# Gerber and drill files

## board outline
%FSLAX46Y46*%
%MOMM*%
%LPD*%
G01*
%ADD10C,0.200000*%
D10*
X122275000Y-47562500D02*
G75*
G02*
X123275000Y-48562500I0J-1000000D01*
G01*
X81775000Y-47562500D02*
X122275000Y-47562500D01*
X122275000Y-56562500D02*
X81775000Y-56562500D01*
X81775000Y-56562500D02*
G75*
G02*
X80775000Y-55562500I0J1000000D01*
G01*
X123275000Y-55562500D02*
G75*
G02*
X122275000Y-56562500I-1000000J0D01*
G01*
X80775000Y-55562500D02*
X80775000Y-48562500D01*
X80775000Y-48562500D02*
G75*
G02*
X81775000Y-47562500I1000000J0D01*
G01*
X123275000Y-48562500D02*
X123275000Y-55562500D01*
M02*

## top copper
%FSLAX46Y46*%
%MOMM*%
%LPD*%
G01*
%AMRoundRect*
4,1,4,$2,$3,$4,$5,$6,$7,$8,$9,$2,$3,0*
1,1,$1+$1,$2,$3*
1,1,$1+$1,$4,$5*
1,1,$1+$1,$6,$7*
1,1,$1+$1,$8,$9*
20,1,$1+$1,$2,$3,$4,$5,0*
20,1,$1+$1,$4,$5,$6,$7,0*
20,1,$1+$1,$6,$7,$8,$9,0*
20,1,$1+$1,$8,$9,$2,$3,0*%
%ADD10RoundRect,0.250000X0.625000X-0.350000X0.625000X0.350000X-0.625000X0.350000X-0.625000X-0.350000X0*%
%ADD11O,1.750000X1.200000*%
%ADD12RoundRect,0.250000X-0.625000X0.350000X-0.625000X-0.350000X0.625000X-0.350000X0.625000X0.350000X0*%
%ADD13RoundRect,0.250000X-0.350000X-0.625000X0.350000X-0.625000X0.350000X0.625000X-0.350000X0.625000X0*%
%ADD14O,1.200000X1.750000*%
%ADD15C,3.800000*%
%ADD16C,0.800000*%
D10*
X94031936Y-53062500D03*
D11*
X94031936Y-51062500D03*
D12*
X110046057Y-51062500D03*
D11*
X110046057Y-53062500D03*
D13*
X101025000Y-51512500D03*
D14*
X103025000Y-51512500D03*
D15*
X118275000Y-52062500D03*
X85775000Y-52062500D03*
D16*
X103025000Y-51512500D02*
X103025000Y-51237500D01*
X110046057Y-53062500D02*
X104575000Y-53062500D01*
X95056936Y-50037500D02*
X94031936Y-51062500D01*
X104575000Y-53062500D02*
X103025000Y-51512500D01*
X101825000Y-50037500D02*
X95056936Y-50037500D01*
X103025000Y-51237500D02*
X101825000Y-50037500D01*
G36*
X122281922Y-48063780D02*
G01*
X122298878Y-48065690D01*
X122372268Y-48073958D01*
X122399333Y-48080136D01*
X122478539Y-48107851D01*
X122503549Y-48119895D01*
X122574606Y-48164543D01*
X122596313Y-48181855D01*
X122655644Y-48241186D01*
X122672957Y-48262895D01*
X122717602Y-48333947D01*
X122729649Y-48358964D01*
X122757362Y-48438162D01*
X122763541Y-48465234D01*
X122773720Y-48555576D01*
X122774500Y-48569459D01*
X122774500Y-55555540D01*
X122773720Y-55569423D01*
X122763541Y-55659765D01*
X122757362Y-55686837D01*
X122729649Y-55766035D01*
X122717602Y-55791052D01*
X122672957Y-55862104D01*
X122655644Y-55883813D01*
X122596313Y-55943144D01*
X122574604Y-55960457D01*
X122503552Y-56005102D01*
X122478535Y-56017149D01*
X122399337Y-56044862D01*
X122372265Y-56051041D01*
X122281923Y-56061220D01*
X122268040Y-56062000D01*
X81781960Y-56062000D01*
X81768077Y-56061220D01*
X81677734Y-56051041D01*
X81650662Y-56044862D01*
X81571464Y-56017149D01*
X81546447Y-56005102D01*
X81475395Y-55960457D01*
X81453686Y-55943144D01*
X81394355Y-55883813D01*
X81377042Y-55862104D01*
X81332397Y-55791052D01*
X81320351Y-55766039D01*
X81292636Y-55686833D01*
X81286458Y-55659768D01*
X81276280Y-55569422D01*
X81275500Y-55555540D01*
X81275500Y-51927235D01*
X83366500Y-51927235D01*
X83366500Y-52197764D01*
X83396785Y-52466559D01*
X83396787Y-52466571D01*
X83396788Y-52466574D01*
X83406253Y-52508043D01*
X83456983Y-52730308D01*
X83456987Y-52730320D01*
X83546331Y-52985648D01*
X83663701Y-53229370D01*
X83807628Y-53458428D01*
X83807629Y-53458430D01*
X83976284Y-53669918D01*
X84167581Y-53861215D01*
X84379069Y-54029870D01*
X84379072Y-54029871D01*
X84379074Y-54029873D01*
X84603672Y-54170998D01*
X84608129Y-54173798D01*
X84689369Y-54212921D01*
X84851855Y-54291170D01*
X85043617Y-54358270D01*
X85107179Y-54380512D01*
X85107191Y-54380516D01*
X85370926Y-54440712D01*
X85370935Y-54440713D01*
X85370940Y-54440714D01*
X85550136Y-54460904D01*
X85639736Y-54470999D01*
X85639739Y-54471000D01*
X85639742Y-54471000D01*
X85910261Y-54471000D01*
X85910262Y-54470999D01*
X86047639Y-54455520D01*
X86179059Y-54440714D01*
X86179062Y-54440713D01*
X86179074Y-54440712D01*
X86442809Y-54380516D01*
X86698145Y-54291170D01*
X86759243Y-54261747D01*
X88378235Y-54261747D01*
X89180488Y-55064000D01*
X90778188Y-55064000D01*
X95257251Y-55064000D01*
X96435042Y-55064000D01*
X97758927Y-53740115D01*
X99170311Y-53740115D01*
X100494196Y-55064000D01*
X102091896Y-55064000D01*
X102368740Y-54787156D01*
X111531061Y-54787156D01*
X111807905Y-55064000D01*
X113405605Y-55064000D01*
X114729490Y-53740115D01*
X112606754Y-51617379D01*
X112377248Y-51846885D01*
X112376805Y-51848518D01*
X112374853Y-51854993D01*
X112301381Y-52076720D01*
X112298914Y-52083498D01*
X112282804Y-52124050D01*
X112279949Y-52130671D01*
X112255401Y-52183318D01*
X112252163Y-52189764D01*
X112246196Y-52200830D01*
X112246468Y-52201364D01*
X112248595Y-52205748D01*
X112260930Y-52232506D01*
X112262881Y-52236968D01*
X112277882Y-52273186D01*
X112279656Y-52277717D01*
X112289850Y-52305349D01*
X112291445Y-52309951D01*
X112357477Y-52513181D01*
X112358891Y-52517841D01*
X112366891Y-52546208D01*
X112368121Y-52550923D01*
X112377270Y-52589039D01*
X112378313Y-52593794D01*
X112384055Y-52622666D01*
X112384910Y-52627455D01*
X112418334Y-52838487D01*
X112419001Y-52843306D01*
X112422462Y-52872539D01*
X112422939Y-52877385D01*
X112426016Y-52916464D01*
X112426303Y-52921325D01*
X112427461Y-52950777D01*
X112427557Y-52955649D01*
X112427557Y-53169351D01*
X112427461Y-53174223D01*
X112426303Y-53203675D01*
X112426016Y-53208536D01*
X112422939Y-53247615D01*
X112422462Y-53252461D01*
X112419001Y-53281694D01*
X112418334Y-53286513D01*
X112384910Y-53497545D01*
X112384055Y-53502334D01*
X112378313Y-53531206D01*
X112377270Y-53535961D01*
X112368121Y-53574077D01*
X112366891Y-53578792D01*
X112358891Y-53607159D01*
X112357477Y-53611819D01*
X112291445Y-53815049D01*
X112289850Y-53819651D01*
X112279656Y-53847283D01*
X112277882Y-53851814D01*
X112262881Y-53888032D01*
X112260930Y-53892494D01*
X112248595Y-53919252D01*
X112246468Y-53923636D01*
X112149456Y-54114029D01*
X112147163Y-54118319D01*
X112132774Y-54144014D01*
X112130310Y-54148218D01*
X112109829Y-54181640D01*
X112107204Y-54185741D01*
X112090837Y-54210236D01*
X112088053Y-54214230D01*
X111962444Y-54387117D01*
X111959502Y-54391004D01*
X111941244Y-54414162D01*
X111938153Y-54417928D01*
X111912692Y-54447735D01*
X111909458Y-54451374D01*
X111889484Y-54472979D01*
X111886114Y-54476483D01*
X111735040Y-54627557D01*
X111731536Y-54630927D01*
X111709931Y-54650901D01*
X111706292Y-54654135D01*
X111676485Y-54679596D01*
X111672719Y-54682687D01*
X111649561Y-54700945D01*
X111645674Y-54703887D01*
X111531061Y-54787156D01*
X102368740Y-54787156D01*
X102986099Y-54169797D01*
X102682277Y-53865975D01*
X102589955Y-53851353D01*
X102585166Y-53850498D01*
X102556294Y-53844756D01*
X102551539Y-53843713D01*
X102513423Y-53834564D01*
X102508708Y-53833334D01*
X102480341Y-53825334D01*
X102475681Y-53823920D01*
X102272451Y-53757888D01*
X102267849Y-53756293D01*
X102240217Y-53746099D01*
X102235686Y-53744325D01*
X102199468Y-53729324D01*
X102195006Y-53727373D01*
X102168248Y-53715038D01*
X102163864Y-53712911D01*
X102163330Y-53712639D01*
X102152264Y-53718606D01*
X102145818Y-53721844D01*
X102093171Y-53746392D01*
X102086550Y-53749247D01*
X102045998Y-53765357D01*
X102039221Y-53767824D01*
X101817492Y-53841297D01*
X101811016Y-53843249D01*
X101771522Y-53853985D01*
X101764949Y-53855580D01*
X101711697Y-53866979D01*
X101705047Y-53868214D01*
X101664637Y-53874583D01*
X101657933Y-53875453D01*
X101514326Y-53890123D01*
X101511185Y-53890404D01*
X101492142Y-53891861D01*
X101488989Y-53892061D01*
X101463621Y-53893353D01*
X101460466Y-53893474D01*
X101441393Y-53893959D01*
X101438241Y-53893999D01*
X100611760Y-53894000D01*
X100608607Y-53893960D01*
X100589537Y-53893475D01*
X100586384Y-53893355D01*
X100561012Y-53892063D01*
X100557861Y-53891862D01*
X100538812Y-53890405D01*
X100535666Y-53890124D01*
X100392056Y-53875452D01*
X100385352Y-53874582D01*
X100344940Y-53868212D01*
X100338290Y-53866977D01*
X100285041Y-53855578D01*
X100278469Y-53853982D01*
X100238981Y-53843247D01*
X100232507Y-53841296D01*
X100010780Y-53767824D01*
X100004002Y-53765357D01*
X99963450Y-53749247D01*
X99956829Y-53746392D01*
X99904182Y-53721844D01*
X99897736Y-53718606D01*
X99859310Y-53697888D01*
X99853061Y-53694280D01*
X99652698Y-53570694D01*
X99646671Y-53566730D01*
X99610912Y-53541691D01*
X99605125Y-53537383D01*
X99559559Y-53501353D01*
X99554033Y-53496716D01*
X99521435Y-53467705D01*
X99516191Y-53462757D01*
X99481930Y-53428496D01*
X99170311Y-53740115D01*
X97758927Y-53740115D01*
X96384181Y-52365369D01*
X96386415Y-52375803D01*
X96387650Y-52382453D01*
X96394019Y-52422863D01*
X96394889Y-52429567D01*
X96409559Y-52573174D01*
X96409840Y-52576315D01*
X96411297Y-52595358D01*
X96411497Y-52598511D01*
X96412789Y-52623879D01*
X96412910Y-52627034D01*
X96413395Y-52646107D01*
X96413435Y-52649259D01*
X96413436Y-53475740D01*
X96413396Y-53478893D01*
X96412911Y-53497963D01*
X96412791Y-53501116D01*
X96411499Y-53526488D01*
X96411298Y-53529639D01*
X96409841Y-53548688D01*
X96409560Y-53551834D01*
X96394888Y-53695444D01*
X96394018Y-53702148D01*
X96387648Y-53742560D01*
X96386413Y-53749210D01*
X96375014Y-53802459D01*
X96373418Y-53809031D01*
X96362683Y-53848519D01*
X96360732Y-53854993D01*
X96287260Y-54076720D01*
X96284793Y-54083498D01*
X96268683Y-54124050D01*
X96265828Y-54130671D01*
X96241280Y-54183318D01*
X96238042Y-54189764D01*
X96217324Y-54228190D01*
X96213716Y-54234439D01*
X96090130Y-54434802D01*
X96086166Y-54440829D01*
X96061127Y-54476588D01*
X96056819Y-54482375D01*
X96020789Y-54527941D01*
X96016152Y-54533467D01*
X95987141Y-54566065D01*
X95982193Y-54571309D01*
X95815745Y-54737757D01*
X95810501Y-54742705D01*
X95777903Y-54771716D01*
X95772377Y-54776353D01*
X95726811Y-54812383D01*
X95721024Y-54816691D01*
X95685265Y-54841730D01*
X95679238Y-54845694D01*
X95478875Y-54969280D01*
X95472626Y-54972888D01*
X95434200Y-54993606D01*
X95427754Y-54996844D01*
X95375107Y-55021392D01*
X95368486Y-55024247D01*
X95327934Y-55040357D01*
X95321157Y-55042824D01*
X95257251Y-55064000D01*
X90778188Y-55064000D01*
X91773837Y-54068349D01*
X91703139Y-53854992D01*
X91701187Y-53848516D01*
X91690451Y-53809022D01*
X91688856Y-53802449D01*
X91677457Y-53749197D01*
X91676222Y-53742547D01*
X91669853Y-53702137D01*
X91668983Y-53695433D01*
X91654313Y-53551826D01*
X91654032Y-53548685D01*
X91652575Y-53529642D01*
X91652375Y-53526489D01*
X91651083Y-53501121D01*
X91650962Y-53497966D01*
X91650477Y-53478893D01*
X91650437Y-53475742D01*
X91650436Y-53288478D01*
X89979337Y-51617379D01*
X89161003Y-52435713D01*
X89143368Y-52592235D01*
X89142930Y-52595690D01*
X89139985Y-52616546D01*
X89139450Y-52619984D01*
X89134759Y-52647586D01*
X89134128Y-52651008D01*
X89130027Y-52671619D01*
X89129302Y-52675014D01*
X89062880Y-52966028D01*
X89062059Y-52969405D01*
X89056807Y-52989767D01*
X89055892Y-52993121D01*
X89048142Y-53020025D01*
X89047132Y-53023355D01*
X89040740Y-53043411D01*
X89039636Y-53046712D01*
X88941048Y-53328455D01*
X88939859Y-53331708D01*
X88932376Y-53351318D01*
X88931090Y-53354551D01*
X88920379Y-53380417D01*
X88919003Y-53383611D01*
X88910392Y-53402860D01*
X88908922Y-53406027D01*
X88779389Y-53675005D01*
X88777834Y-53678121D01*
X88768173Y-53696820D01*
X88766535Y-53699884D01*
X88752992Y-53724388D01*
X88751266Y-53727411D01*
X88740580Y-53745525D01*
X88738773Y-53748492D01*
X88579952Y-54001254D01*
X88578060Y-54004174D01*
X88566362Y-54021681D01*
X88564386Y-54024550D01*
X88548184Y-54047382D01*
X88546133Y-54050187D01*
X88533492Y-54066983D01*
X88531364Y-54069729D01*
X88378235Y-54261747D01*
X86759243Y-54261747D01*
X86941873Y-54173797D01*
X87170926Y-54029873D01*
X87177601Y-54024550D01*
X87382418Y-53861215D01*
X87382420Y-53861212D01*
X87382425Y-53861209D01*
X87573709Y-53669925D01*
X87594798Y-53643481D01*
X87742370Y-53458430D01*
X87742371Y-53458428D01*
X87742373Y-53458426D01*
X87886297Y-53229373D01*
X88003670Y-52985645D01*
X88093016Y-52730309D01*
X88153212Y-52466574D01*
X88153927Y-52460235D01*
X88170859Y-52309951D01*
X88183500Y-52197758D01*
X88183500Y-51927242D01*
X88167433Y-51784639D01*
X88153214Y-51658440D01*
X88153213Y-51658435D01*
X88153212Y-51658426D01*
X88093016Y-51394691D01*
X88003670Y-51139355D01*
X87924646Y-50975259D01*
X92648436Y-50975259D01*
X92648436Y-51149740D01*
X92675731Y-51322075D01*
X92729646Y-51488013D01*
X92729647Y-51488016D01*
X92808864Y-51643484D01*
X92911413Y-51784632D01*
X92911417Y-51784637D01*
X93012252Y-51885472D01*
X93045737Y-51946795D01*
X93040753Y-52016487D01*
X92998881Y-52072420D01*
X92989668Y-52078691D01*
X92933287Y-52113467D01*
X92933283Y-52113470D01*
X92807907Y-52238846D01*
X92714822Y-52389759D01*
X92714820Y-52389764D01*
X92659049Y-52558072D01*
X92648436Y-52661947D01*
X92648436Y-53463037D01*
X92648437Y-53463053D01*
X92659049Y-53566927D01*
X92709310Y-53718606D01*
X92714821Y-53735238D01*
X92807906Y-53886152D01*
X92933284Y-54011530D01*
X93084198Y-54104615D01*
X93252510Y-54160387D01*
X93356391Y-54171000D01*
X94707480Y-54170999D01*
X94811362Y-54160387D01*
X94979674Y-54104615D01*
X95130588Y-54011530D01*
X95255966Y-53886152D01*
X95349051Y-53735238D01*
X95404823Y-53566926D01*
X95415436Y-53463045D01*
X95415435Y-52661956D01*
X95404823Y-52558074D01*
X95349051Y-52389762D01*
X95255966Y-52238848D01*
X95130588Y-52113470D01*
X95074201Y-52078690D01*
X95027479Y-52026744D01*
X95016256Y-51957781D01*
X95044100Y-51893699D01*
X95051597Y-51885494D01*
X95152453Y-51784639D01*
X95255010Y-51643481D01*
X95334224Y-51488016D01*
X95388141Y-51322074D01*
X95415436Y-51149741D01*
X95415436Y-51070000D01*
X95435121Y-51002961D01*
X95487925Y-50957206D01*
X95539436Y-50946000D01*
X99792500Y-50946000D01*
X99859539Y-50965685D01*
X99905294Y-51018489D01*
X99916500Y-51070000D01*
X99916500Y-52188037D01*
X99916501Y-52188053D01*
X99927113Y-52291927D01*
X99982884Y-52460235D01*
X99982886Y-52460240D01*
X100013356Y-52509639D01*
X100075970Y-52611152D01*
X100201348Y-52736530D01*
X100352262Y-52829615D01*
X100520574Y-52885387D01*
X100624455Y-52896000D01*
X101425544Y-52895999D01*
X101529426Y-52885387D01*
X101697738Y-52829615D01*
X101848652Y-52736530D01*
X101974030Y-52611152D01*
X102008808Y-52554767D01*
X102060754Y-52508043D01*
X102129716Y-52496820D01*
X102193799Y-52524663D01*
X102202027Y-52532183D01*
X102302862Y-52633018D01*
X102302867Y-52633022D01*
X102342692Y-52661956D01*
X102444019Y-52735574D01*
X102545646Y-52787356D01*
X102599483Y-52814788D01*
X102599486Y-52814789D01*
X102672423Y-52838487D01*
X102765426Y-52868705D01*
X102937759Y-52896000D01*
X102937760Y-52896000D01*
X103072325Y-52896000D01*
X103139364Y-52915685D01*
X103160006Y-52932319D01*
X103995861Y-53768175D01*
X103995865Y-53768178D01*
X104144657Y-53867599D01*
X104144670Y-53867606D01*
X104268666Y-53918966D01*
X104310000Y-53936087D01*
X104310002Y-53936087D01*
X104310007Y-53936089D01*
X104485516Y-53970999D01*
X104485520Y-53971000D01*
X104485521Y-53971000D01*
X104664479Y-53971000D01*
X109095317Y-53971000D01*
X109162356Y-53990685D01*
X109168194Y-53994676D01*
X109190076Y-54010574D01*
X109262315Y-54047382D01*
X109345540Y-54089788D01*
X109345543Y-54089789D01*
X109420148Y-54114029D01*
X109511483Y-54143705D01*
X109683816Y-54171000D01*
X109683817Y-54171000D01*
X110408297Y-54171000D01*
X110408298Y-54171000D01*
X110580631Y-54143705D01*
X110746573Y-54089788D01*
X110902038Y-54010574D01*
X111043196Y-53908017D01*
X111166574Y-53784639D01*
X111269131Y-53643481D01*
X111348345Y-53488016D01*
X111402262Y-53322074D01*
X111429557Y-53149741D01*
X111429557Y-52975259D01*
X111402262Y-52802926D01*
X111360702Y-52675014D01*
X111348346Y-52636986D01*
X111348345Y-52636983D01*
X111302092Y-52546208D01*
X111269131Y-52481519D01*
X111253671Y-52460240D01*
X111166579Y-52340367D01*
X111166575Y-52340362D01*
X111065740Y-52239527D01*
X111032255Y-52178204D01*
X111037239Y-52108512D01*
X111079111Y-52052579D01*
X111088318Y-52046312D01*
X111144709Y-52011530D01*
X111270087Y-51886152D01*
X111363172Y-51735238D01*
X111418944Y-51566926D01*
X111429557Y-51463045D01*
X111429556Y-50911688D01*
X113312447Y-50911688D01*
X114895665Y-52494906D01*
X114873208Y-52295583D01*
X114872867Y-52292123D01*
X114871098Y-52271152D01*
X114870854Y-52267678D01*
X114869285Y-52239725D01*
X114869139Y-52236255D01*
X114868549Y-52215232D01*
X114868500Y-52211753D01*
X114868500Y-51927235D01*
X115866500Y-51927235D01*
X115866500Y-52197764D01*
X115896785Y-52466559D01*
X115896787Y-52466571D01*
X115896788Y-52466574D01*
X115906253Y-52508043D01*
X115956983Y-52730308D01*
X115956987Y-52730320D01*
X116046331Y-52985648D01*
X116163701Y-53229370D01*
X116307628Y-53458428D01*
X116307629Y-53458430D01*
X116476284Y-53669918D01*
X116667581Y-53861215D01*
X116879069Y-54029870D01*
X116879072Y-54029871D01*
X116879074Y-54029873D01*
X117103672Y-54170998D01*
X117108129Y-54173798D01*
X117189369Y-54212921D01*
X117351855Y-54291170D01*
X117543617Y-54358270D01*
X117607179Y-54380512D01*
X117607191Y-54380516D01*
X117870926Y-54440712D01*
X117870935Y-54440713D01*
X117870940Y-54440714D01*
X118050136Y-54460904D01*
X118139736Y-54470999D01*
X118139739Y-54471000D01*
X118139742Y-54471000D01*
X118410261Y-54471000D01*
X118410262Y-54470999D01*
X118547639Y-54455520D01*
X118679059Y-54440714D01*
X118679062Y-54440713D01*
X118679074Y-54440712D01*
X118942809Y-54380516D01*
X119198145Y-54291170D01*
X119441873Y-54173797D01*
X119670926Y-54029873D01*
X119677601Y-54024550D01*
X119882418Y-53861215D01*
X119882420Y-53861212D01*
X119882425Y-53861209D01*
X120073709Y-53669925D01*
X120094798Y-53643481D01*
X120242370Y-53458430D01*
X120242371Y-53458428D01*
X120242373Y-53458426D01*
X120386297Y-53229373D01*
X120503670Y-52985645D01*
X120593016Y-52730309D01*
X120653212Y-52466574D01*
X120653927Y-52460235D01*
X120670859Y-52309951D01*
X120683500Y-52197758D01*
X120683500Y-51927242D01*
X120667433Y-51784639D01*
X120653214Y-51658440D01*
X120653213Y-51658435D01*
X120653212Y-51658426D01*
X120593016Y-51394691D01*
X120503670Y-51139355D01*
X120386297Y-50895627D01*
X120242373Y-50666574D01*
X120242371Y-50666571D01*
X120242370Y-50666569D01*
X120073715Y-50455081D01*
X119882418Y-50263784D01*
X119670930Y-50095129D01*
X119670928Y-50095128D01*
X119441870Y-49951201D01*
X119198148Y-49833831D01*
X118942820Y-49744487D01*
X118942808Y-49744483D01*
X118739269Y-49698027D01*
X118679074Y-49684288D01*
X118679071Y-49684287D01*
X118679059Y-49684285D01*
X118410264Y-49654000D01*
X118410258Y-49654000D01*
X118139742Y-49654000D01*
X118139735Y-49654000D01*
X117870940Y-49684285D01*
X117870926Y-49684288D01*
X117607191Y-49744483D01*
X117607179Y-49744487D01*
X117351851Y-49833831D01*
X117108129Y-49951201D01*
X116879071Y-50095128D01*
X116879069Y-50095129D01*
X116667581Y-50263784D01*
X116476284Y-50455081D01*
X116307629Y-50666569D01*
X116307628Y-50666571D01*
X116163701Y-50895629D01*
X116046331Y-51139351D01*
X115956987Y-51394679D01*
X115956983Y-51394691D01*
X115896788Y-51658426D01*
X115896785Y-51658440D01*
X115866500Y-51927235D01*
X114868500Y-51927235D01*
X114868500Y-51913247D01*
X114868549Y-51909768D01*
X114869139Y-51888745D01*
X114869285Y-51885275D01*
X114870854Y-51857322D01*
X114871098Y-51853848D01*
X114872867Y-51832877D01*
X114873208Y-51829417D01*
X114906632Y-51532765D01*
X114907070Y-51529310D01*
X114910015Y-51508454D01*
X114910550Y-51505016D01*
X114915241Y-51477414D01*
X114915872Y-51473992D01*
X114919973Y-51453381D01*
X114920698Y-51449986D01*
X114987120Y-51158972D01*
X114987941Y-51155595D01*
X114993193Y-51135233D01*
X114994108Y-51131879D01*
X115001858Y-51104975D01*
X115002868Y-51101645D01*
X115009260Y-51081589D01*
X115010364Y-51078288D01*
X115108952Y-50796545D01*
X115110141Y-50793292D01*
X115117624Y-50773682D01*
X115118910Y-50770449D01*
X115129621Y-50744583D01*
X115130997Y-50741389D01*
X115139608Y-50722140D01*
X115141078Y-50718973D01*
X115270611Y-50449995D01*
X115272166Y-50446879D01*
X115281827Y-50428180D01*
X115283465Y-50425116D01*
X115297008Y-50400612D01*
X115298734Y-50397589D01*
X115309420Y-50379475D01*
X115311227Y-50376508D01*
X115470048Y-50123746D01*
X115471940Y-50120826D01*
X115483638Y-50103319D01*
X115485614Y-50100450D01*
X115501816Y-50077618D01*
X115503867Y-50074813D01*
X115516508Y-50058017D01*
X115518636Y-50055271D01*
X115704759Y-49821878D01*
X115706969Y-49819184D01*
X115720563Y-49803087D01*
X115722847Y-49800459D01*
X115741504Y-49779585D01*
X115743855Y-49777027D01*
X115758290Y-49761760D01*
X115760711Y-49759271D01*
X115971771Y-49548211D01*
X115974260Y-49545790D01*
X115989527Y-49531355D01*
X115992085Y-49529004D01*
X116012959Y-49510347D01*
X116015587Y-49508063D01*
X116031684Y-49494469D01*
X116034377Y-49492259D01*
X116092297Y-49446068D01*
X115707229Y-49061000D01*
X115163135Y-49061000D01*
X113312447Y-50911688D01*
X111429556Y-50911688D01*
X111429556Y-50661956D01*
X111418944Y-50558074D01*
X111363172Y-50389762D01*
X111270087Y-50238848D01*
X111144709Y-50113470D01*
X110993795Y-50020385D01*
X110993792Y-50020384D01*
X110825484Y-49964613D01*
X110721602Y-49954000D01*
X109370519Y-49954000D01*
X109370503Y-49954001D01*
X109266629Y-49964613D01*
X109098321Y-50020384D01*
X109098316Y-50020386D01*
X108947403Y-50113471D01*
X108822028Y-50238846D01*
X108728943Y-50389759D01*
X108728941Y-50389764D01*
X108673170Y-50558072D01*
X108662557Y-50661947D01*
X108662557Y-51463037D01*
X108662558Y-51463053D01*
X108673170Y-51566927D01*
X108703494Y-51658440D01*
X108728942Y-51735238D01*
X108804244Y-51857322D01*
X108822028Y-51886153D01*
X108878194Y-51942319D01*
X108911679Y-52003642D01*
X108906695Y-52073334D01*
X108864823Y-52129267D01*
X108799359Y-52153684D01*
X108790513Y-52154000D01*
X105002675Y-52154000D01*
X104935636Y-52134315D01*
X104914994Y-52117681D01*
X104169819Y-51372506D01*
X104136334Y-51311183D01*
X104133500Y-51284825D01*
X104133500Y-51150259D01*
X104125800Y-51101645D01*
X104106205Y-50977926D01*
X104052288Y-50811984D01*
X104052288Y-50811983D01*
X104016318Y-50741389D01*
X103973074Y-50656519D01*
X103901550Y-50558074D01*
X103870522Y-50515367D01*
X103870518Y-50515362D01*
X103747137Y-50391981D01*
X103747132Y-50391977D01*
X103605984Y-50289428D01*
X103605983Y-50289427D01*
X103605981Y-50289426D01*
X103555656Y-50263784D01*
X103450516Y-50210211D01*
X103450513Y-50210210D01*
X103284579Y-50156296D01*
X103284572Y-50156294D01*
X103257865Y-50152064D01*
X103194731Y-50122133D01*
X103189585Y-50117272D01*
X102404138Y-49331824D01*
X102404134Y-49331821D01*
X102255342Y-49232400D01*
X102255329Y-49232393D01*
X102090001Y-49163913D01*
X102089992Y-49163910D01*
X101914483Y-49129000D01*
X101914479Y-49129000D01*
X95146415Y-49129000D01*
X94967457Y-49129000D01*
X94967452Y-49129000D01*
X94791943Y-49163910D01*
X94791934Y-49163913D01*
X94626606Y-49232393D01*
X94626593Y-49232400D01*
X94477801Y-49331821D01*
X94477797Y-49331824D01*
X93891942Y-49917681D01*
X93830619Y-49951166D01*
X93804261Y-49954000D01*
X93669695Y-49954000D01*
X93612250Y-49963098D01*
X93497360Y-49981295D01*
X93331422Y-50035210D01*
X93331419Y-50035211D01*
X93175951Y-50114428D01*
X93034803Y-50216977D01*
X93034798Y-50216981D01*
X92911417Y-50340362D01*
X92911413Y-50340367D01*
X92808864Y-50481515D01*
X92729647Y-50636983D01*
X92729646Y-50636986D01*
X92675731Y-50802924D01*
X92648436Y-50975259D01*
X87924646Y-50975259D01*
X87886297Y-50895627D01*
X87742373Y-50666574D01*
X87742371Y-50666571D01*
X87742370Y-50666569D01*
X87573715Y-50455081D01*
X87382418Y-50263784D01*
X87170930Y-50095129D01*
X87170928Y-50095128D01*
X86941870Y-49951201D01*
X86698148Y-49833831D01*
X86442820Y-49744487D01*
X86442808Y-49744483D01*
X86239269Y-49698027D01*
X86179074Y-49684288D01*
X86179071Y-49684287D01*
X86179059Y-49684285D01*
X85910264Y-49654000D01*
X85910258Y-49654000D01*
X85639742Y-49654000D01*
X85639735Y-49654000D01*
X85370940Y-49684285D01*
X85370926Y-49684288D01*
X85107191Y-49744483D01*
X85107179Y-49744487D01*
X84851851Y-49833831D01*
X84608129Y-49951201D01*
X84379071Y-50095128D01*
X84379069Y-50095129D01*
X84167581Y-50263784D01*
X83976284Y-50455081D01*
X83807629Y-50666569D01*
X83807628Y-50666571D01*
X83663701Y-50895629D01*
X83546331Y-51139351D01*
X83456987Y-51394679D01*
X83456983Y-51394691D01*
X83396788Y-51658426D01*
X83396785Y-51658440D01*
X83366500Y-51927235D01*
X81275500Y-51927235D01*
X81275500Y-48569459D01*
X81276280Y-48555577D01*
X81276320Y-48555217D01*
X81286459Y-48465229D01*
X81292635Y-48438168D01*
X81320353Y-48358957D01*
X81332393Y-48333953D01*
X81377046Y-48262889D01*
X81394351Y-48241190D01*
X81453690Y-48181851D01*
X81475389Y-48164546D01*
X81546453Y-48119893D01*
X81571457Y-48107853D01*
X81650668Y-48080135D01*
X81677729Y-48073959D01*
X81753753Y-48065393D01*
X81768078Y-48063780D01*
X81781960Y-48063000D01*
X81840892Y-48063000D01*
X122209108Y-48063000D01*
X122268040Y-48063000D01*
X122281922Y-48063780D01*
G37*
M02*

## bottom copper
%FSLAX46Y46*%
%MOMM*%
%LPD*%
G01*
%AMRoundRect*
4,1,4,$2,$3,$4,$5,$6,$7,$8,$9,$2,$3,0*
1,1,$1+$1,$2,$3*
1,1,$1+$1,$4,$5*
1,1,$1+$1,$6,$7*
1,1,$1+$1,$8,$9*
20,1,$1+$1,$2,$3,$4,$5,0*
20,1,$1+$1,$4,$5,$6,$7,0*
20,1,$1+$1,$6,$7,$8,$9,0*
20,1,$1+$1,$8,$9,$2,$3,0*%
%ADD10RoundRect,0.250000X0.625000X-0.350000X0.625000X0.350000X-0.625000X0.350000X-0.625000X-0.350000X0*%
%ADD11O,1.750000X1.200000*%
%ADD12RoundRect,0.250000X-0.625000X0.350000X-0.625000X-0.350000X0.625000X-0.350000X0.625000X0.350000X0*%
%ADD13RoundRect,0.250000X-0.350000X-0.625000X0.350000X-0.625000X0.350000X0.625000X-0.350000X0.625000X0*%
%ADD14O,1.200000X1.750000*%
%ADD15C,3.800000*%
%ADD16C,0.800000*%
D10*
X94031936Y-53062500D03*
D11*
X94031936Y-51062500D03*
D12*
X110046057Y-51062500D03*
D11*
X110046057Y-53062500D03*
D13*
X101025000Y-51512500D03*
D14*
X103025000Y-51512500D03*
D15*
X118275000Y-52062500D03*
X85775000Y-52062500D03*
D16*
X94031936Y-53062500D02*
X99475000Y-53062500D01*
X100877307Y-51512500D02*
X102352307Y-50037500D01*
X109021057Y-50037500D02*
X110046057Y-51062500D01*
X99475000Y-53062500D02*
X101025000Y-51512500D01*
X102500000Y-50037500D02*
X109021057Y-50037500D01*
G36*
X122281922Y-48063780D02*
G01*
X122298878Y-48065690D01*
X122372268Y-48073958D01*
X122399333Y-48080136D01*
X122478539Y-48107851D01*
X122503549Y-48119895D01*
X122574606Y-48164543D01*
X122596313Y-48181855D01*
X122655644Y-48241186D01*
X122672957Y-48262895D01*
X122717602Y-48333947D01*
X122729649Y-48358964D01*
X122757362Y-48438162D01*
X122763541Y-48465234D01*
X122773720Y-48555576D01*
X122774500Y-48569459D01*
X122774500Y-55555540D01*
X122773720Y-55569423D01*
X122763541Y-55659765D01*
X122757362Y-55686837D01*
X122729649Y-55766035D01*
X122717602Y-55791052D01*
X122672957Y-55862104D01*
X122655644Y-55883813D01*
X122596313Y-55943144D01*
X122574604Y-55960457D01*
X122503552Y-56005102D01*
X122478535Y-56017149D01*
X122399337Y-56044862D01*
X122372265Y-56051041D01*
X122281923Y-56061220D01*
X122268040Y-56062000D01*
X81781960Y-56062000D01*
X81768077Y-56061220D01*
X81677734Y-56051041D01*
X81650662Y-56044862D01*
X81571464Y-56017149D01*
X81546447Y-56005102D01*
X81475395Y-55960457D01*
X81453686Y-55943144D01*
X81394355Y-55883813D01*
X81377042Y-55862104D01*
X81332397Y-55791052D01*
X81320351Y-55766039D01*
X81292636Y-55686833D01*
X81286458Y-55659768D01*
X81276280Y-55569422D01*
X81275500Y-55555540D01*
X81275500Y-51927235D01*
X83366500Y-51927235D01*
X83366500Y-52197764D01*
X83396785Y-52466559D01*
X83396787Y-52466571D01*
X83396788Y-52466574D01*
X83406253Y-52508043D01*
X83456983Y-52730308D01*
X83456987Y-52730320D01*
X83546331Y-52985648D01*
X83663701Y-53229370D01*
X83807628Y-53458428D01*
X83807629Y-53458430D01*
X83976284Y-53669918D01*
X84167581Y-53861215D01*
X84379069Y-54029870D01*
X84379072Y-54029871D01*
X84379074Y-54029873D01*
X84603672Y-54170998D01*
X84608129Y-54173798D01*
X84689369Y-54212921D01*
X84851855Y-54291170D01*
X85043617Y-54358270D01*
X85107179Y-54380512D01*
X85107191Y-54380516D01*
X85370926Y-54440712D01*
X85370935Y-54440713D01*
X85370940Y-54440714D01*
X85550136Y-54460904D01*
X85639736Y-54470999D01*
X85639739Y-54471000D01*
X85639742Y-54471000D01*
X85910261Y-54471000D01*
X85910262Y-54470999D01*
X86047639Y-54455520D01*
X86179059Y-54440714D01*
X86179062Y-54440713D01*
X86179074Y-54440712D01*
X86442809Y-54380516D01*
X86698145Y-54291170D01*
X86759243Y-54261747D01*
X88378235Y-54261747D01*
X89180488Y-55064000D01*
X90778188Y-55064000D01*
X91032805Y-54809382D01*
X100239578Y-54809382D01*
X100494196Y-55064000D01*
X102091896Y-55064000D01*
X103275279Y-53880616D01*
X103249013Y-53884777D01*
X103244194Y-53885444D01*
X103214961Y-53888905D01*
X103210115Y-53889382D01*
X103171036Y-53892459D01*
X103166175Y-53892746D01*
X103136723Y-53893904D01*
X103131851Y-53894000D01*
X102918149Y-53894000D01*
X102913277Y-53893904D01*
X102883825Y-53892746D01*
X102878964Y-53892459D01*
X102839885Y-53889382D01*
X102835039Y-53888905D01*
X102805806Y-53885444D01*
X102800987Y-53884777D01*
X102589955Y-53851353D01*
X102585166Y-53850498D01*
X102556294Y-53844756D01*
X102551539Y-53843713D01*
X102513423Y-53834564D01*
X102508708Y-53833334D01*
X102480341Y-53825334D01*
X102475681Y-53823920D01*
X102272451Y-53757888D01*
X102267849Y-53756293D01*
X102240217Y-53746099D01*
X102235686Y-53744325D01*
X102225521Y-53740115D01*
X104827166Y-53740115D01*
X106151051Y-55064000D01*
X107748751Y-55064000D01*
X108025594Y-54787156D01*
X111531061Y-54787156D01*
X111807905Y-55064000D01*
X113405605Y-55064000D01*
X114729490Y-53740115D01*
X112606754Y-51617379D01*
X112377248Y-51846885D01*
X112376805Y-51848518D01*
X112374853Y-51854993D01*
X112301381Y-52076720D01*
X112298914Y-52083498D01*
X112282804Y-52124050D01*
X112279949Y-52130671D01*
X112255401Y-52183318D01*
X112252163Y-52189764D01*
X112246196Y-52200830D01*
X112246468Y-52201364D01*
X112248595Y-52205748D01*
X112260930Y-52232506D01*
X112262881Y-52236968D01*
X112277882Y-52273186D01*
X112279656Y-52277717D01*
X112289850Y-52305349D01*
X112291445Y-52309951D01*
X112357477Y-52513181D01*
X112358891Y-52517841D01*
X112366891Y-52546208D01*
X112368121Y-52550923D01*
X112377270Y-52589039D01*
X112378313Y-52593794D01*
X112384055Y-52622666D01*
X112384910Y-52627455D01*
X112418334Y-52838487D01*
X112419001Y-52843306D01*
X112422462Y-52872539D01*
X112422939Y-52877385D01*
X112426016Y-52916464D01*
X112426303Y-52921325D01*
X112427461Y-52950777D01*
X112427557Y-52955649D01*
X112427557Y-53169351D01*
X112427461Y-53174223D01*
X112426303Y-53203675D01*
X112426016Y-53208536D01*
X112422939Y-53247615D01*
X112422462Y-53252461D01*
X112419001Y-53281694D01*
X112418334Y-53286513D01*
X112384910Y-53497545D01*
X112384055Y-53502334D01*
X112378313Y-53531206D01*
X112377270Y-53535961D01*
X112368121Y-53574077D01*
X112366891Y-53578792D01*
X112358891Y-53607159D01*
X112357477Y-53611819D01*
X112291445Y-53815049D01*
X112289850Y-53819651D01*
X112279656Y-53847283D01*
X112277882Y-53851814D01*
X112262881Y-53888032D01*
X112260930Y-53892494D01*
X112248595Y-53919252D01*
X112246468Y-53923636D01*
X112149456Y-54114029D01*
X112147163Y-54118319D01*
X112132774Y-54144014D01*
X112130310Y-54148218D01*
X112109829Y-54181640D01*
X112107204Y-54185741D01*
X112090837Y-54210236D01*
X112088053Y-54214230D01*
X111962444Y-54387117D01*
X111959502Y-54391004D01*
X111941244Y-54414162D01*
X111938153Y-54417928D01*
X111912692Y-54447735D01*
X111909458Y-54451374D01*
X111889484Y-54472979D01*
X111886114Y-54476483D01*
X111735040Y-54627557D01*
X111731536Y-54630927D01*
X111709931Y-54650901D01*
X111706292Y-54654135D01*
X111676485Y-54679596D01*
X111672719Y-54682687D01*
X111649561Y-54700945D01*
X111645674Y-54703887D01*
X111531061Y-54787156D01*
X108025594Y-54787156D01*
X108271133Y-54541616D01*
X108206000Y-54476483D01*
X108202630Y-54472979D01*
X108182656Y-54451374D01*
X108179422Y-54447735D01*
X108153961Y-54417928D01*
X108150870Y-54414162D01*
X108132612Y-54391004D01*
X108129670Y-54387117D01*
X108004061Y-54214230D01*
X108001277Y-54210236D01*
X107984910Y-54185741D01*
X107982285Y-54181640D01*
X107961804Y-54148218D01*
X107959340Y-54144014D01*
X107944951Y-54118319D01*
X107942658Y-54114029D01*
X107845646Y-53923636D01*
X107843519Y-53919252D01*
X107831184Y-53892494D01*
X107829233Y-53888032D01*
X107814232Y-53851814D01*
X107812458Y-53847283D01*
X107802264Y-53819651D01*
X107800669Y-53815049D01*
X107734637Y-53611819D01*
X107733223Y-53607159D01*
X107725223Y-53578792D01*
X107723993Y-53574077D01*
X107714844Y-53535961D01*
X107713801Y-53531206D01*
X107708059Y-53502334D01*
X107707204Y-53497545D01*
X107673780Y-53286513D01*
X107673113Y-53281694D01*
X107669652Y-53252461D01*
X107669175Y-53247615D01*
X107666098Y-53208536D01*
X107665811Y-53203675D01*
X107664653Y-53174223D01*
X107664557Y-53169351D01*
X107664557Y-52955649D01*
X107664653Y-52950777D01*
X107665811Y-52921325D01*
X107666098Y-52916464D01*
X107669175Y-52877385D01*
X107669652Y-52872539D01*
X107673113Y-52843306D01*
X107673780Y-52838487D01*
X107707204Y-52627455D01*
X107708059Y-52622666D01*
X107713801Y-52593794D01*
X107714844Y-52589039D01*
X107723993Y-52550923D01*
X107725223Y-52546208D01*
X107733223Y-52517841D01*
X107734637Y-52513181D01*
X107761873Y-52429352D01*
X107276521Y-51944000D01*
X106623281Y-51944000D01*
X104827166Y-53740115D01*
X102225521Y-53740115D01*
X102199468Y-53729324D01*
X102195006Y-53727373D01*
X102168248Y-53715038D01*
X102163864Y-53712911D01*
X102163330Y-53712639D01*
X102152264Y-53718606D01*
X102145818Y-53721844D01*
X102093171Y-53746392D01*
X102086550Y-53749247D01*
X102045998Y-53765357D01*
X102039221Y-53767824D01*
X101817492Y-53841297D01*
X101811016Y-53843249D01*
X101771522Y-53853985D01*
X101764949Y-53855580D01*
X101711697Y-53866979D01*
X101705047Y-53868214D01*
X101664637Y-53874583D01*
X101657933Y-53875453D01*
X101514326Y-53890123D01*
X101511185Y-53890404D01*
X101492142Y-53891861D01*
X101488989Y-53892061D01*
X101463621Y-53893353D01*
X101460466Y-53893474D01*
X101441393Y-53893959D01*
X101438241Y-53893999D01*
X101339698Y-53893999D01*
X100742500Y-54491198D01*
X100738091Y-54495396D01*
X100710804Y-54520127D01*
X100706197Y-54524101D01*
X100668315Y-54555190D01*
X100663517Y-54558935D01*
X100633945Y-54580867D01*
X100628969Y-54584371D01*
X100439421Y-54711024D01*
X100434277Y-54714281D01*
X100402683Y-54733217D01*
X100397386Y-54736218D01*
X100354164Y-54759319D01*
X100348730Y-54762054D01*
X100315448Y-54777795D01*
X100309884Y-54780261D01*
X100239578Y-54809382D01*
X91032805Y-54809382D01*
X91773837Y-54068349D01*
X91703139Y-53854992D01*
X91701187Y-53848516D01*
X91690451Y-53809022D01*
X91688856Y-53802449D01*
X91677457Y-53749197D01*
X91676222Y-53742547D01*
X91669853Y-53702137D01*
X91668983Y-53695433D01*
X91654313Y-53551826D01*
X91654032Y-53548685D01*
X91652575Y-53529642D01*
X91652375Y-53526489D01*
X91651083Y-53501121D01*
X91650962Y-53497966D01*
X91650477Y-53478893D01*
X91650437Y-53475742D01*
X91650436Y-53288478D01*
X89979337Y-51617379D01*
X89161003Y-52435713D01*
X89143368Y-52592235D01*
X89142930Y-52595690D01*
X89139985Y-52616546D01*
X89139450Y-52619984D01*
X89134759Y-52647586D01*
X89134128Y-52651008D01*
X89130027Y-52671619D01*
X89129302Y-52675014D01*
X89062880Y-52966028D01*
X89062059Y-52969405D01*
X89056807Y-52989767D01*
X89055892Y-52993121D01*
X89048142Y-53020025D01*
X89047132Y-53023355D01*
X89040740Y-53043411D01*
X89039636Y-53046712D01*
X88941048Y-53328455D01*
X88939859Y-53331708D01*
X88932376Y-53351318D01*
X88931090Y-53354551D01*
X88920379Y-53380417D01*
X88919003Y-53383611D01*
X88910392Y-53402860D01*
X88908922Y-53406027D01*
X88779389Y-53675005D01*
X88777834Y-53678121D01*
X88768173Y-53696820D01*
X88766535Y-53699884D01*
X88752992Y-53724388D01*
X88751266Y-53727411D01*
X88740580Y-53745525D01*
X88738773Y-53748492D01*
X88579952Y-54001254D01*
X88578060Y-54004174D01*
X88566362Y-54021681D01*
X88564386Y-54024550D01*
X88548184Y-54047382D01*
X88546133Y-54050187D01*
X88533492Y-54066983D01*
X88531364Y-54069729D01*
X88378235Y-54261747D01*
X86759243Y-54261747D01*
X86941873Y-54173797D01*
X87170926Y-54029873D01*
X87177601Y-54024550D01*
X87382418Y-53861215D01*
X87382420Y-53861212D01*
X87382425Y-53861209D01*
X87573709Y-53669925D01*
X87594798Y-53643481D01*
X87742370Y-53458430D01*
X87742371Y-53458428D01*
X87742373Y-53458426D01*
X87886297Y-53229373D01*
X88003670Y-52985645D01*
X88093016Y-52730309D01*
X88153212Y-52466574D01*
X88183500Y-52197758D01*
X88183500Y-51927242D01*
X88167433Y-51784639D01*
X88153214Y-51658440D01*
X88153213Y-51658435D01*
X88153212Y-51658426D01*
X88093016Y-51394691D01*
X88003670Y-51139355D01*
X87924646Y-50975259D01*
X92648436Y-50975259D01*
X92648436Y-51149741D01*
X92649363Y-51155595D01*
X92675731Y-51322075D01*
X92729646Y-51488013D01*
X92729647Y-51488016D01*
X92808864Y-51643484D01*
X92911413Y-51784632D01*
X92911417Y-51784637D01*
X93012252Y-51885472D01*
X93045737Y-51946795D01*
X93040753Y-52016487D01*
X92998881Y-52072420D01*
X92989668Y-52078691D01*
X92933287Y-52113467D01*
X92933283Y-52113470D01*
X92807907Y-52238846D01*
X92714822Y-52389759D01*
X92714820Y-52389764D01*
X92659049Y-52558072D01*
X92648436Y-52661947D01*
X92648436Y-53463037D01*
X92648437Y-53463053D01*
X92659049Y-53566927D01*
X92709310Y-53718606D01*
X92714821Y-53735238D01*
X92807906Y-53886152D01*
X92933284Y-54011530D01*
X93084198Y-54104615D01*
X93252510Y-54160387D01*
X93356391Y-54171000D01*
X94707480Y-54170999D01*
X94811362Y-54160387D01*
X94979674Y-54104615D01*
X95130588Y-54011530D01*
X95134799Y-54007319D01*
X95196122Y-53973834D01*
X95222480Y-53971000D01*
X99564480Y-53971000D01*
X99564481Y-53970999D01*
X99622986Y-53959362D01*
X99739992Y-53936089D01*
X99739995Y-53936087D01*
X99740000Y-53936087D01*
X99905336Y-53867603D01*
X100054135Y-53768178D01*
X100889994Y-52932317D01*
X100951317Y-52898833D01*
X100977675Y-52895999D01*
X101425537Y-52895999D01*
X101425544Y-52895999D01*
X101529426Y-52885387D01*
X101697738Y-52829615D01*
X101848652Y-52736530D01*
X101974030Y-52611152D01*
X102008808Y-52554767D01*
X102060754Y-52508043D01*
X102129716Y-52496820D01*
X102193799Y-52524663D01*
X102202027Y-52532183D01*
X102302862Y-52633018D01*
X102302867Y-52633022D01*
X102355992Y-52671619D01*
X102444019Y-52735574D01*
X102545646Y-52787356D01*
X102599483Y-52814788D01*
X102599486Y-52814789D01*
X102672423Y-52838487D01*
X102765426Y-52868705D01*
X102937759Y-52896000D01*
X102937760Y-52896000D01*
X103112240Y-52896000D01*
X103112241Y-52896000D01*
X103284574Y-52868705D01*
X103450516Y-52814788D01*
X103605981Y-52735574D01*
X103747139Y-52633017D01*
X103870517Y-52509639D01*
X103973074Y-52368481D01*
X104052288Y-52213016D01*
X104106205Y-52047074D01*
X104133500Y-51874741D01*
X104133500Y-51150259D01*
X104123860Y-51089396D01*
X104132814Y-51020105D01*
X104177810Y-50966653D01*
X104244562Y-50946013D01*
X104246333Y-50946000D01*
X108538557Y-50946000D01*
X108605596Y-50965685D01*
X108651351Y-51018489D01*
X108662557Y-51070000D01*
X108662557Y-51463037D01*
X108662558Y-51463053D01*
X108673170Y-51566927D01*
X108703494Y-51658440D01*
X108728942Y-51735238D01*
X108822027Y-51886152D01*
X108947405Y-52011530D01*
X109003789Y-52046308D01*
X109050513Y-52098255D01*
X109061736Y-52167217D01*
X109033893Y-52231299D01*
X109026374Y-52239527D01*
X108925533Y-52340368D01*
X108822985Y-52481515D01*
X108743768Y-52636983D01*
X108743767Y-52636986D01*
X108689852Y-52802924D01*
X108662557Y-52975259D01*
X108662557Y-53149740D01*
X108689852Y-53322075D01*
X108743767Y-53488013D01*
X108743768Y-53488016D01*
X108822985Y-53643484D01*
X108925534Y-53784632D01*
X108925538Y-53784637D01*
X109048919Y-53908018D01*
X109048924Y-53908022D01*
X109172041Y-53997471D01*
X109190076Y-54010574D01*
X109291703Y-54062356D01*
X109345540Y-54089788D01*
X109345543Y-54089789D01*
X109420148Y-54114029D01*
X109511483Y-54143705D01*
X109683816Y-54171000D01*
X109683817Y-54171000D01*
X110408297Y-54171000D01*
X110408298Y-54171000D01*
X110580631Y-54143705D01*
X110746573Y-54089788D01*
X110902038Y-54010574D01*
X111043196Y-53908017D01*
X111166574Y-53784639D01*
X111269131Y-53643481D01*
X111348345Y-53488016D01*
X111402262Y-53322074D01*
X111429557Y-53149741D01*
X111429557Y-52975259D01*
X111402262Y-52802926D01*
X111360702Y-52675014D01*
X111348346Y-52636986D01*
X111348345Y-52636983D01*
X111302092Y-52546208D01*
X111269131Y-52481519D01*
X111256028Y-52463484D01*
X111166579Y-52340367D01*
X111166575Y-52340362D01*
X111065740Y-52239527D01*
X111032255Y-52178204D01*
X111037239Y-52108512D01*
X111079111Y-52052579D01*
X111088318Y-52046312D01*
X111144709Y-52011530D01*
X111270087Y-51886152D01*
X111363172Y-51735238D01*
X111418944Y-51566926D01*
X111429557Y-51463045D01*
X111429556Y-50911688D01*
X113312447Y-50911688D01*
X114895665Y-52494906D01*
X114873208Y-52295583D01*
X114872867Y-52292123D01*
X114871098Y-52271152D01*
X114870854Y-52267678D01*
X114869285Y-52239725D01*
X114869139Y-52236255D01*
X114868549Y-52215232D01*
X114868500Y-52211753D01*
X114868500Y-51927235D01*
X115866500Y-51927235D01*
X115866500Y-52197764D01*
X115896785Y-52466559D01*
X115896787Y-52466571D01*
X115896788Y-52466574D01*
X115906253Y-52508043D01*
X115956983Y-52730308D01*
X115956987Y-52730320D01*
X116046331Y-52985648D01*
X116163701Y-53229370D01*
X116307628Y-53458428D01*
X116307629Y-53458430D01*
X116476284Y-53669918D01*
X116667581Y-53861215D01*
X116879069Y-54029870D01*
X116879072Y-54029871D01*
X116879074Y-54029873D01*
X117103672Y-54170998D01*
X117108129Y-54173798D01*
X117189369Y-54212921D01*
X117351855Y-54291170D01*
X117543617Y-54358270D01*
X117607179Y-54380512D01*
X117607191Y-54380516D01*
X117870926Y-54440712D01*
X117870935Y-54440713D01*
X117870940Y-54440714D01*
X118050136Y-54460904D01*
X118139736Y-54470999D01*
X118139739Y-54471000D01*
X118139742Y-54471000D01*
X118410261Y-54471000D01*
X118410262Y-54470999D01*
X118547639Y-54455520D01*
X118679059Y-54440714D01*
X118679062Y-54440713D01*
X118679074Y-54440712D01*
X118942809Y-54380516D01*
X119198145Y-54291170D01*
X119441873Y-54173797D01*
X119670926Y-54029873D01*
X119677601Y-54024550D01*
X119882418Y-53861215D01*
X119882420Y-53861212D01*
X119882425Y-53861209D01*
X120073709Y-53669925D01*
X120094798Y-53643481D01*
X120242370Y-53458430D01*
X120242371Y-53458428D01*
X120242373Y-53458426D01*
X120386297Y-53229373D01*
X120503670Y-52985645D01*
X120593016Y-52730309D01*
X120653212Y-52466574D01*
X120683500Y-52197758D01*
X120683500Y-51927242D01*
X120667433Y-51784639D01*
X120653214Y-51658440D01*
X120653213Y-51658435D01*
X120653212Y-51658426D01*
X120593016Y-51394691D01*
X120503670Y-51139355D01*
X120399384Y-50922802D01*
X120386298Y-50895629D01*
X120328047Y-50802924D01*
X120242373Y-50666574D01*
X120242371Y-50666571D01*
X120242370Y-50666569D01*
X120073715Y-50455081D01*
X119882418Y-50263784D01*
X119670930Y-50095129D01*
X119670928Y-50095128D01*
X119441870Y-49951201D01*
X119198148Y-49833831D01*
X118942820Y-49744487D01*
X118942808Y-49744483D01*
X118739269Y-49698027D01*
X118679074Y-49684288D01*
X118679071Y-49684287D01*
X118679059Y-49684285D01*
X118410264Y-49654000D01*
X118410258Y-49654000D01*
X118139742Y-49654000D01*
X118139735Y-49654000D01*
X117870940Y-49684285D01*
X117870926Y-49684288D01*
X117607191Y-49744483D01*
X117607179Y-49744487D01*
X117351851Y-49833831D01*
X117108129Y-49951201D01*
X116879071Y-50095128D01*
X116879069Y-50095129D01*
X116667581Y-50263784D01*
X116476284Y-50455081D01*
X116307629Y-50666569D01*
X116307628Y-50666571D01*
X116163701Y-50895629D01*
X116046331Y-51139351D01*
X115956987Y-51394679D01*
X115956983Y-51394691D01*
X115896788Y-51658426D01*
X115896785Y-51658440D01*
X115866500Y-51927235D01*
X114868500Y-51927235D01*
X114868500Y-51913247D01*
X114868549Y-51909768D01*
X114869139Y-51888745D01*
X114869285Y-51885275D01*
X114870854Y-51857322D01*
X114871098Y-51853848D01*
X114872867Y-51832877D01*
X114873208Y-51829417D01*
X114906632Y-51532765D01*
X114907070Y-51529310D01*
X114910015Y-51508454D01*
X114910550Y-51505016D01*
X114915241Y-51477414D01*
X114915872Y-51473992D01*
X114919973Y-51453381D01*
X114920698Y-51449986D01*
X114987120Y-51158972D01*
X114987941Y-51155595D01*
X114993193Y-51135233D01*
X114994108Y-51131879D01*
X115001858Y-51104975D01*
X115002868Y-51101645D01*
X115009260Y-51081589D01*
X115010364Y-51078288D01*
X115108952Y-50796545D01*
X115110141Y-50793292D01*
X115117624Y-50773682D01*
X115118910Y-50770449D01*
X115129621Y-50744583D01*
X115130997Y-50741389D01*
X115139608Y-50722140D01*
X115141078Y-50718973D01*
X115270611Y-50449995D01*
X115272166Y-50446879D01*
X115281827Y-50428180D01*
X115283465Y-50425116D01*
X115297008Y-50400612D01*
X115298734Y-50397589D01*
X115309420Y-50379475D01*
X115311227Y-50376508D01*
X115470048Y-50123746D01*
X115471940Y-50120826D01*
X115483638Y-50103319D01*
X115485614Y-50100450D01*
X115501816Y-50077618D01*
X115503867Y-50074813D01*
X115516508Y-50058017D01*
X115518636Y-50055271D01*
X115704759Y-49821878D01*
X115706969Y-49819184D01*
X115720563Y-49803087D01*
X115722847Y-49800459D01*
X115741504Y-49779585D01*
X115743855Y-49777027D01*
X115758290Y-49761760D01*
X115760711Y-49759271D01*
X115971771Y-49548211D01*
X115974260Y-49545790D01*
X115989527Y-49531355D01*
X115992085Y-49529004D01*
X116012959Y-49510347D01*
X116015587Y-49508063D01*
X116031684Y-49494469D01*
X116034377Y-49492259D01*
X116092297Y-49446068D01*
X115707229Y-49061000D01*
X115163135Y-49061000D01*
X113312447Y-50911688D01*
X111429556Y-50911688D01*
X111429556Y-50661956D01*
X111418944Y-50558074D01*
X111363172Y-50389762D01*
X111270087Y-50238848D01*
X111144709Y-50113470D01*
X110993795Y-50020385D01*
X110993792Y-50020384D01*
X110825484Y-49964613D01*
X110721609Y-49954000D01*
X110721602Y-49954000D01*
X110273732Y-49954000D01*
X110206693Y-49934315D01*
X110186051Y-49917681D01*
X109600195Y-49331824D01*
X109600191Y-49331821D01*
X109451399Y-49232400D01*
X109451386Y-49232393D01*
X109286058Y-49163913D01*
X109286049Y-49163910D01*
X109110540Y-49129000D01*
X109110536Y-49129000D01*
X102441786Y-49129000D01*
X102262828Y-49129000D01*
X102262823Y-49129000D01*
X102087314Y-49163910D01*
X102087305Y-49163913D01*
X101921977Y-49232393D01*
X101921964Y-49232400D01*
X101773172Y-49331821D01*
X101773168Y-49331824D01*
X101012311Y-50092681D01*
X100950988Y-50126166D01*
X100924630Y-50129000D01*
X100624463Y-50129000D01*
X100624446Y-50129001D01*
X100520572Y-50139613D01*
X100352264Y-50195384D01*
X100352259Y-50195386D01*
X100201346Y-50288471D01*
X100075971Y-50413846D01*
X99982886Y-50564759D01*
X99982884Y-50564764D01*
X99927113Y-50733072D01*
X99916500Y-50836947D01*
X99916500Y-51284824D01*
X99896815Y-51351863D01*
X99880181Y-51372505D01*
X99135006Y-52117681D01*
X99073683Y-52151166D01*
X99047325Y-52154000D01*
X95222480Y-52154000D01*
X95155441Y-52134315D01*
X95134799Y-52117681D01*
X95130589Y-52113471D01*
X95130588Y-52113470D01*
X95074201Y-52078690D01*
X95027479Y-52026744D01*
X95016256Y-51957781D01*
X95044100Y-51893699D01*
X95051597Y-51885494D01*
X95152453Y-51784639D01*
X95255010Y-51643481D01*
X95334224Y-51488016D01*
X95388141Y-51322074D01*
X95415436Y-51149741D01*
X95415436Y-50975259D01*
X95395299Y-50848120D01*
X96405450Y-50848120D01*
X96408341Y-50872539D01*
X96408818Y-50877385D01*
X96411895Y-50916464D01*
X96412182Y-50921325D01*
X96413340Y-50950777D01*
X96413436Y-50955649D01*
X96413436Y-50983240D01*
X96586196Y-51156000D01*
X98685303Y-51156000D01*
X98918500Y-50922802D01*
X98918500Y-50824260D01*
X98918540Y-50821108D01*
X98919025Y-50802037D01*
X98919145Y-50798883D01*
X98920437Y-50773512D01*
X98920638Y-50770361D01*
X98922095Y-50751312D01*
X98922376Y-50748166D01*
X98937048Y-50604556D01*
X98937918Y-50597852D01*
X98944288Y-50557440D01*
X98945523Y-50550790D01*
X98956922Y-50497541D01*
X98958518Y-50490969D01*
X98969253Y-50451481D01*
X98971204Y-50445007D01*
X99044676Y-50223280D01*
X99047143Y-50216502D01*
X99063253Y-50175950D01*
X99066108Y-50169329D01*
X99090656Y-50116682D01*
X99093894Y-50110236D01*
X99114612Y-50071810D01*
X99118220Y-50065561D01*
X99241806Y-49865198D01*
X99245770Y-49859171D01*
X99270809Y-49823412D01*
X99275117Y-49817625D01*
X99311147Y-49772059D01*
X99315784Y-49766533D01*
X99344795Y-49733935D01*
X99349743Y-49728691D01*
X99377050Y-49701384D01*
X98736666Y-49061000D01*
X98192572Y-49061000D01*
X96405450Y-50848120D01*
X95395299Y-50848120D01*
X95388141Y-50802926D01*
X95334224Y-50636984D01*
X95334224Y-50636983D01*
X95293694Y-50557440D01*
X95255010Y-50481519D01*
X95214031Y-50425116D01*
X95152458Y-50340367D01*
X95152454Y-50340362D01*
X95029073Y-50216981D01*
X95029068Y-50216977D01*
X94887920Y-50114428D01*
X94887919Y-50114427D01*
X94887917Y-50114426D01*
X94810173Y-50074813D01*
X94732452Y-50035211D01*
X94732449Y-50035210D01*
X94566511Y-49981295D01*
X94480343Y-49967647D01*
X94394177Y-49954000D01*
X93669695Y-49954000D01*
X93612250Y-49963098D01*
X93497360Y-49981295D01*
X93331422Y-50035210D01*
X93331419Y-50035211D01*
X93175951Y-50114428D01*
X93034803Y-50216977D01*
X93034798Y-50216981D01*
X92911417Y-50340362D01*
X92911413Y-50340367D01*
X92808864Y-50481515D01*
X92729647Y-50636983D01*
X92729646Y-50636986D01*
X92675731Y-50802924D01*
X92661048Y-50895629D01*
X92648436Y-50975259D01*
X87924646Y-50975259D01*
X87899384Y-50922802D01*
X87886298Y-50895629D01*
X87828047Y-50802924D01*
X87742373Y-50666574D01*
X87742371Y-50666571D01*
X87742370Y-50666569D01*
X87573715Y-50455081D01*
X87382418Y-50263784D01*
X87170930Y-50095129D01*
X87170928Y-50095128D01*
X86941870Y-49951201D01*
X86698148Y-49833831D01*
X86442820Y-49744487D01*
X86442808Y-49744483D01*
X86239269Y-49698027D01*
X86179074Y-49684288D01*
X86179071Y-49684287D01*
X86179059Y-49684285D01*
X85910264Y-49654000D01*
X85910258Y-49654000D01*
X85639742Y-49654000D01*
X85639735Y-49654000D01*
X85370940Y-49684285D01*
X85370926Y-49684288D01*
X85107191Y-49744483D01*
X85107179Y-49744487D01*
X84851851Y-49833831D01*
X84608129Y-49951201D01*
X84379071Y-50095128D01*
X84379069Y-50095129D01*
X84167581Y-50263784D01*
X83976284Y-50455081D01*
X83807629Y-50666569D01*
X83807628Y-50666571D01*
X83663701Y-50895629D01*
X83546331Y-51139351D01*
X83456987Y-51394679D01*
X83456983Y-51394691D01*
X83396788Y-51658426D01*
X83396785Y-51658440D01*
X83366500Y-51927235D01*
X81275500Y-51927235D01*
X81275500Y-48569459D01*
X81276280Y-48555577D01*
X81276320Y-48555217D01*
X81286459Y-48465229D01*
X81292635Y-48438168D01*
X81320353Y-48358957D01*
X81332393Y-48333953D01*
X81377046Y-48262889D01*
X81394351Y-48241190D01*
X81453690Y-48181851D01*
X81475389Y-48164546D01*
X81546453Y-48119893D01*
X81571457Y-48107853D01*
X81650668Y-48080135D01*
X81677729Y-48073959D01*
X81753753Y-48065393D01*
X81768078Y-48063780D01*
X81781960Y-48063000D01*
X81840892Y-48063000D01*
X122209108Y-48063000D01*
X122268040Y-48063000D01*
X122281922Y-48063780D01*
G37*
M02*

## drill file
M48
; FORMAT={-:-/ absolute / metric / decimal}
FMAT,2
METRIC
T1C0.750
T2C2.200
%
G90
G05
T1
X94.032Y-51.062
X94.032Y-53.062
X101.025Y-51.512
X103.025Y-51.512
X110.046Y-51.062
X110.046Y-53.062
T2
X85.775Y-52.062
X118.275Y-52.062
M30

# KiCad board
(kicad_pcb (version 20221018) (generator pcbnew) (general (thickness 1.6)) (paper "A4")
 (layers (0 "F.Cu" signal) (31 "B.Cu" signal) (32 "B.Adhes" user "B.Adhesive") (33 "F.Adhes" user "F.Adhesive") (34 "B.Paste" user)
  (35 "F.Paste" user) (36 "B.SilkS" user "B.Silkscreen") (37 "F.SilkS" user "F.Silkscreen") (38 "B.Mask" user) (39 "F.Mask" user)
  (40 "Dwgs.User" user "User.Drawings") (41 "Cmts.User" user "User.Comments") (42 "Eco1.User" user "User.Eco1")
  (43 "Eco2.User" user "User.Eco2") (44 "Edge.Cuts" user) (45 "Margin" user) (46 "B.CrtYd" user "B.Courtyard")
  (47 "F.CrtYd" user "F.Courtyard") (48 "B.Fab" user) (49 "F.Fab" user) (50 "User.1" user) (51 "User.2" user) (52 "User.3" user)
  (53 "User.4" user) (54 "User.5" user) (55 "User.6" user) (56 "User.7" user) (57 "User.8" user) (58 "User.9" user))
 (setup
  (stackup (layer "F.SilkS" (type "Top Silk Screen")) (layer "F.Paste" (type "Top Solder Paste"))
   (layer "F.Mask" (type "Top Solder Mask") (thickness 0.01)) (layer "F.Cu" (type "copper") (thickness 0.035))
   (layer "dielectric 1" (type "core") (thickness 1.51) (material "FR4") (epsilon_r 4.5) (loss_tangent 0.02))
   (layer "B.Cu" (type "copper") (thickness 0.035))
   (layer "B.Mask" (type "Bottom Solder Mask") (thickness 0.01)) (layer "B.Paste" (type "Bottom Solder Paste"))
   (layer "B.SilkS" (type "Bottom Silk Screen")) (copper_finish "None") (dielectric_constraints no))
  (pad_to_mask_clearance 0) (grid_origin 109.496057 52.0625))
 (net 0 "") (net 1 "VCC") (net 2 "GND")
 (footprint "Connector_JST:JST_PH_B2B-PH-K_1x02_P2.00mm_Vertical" (layer "F.Cu") (at 94.031936 53.0625 90)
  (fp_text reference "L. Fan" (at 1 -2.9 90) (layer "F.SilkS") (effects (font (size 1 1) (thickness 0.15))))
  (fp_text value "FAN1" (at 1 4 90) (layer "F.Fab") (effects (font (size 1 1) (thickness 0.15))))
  (pad "1" thru_hole roundrect (at 0 0 90) (size 1.2 1.75) (drill 0.75) (layers "*.Cu" "*.Mask") (roundrect_rratio 0.2083333333)
   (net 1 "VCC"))
  (pad "2" thru_hole oval (at 2 0 90) (size 1.2 1.75) (drill 0.75) (layers "*.Cu" "*.Mask") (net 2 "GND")))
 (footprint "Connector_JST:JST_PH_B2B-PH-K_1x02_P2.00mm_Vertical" (layer "F.Cu") (at 110.046057 51.0625 -90)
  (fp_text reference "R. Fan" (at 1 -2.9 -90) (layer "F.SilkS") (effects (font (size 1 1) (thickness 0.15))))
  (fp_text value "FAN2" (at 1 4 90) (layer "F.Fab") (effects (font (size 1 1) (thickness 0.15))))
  (pad "1" thru_hole roundrect (at 0 0 270) (size 1.2 1.75) (drill 0.75) (layers "*.Cu" "*.Mask") (roundrect_rratio 0.2083333333)
   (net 1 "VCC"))
  (pad "2" thru_hole oval (at 2 0 270) (size 1.2 1.75) (drill 0.75) (layers "*.Cu" "*.Mask") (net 2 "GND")))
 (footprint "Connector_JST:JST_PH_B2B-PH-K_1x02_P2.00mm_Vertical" (layer "F.Cu") (at 101.025 51.5125)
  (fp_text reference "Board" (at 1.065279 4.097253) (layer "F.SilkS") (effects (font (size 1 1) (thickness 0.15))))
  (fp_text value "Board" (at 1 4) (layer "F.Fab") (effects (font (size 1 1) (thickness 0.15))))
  (pad "1" thru_hole roundrect (at 0 0) (size 1.2 1.75) (drill 0.75) (layers "*.Cu" "*.Mask") (roundrect_rratio 0.2083333333) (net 1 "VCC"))
  (pad "2" thru_hole oval (at 2 0) (size 1.2 1.75) (drill 0.75) (layers "*.Cu" "*.Mask") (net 2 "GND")))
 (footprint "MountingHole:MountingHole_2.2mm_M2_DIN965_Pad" (layer "F.Cu") (at 118.275 52.0625)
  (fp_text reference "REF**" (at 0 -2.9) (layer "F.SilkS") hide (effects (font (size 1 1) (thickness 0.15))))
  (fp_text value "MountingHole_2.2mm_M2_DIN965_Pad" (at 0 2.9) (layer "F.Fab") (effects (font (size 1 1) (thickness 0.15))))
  (pad "1" thru_hole circle (at 0 0) (size 3.8 3.8) (drill 2.2) (layers "*.Cu" "*.Mask")))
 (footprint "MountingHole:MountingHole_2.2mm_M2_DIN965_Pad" (layer "F.Cu") (at 85.775 52.0625)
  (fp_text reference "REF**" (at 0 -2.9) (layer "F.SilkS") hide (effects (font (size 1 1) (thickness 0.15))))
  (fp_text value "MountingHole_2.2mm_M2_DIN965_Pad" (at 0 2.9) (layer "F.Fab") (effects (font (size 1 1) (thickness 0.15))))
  (pad "1" thru_hole circle (at 0 0) (size 3.8 3.8) (drill 2.2) (layers "*.Cu" "*.Mask")))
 (gr_arc (start 122.275 47.5625) (mid 122.982107 47.855393) (end 123.275 48.5625) (stroke (width 0.2) (type solid)) (layer "Edge.Cuts"))
 (gr_line (start 81.775 47.5625) (end 122.275 47.5625) (stroke (width 0.2) (type solid)) (layer "Edge.Cuts"))
 (gr_line (start 122.275 56.5625) (end 81.775 56.5625) (stroke (width 0.2) (type solid)) (layer "Edge.Cuts"))
 (gr_arc (start 81.775 56.5625) (mid 81.067893 56.269607) (end 80.775 55.5625) (stroke (width 0.2) (type solid)) (layer "Edge.Cuts"))
 (gr_arc (start 123.275 55.5625) (mid 122.982107 56.269607) (end 122.275 56.5625) (stroke (width 0.2) (type solid)) (layer "Edge.Cuts"))
 (gr_line (start 80.775 55.5625) (end 80.775 48.5625) (stroke (width 0.2) (type solid)) (layer "Edge.Cuts"))
 (gr_arc (start 80.775 48.5625) (mid 81.067893 47.855393) (end 81.775 47.5625) (stroke (width 0.2) (type solid)) (layer "Edge.Cuts"))
 (gr_line (start 123.275 48.5625) (end 123.275 55.5625) (stroke (width 0.2) (type solid)) (layer "Edge.Cuts"))
 (segment (start 94.031936 53.0625) (end 99.475 53.0625) (width 0.8) (layer "B.Cu") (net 1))
 (segment (start 100.877307 51.5125) (end 102.352307 50.0375) (width 0.8) (layer "B.Cu") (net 1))
 (segment (start 109.021057 50.0375) (end 110.046057 51.0625) (width 0.8) (layer "B.Cu") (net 1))
 (segment (start 99.475 53.0625) (end 101.025 51.5125) (width 0.8) (layer "B.Cu") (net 1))
 (segment (start 102.5 50.0375) (end 109.021057 50.0375) (width 0.8) (layer "B.Cu") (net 1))
 (segment (start 103.025 51.5125) (end 103.025 51.2375) (width 0.8) (layer "F.Cu") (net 2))
 (segment (start 110.046057 53.0625) (end 104.575 53.0625) (width 0.8) (layer "F.Cu") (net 2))
 (segment (start 95.056936 50.0375) (end 94.031936 51.0625) (width 0.8) (layer "F.Cu") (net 2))
 (segment (start 104.575 53.0625) (end 103.025 51.5125) (width 0.8) (layer "F.Cu") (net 2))
 (segment (start 101.825 50.0375) (end 95.056936 50.0375) (width 0.8) (layer "F.Cu") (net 2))
 (segment (start 103.025 51.2375) (end 101.825 50.0375) (width 0.8) (layer "F.Cu") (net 2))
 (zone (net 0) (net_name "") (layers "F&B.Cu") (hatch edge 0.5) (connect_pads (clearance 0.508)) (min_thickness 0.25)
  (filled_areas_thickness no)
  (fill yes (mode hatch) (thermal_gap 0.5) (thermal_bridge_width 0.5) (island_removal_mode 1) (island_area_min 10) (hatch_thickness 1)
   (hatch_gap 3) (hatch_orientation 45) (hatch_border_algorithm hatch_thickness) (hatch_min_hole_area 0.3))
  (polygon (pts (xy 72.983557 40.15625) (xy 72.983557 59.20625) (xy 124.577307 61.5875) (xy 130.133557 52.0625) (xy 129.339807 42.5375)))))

